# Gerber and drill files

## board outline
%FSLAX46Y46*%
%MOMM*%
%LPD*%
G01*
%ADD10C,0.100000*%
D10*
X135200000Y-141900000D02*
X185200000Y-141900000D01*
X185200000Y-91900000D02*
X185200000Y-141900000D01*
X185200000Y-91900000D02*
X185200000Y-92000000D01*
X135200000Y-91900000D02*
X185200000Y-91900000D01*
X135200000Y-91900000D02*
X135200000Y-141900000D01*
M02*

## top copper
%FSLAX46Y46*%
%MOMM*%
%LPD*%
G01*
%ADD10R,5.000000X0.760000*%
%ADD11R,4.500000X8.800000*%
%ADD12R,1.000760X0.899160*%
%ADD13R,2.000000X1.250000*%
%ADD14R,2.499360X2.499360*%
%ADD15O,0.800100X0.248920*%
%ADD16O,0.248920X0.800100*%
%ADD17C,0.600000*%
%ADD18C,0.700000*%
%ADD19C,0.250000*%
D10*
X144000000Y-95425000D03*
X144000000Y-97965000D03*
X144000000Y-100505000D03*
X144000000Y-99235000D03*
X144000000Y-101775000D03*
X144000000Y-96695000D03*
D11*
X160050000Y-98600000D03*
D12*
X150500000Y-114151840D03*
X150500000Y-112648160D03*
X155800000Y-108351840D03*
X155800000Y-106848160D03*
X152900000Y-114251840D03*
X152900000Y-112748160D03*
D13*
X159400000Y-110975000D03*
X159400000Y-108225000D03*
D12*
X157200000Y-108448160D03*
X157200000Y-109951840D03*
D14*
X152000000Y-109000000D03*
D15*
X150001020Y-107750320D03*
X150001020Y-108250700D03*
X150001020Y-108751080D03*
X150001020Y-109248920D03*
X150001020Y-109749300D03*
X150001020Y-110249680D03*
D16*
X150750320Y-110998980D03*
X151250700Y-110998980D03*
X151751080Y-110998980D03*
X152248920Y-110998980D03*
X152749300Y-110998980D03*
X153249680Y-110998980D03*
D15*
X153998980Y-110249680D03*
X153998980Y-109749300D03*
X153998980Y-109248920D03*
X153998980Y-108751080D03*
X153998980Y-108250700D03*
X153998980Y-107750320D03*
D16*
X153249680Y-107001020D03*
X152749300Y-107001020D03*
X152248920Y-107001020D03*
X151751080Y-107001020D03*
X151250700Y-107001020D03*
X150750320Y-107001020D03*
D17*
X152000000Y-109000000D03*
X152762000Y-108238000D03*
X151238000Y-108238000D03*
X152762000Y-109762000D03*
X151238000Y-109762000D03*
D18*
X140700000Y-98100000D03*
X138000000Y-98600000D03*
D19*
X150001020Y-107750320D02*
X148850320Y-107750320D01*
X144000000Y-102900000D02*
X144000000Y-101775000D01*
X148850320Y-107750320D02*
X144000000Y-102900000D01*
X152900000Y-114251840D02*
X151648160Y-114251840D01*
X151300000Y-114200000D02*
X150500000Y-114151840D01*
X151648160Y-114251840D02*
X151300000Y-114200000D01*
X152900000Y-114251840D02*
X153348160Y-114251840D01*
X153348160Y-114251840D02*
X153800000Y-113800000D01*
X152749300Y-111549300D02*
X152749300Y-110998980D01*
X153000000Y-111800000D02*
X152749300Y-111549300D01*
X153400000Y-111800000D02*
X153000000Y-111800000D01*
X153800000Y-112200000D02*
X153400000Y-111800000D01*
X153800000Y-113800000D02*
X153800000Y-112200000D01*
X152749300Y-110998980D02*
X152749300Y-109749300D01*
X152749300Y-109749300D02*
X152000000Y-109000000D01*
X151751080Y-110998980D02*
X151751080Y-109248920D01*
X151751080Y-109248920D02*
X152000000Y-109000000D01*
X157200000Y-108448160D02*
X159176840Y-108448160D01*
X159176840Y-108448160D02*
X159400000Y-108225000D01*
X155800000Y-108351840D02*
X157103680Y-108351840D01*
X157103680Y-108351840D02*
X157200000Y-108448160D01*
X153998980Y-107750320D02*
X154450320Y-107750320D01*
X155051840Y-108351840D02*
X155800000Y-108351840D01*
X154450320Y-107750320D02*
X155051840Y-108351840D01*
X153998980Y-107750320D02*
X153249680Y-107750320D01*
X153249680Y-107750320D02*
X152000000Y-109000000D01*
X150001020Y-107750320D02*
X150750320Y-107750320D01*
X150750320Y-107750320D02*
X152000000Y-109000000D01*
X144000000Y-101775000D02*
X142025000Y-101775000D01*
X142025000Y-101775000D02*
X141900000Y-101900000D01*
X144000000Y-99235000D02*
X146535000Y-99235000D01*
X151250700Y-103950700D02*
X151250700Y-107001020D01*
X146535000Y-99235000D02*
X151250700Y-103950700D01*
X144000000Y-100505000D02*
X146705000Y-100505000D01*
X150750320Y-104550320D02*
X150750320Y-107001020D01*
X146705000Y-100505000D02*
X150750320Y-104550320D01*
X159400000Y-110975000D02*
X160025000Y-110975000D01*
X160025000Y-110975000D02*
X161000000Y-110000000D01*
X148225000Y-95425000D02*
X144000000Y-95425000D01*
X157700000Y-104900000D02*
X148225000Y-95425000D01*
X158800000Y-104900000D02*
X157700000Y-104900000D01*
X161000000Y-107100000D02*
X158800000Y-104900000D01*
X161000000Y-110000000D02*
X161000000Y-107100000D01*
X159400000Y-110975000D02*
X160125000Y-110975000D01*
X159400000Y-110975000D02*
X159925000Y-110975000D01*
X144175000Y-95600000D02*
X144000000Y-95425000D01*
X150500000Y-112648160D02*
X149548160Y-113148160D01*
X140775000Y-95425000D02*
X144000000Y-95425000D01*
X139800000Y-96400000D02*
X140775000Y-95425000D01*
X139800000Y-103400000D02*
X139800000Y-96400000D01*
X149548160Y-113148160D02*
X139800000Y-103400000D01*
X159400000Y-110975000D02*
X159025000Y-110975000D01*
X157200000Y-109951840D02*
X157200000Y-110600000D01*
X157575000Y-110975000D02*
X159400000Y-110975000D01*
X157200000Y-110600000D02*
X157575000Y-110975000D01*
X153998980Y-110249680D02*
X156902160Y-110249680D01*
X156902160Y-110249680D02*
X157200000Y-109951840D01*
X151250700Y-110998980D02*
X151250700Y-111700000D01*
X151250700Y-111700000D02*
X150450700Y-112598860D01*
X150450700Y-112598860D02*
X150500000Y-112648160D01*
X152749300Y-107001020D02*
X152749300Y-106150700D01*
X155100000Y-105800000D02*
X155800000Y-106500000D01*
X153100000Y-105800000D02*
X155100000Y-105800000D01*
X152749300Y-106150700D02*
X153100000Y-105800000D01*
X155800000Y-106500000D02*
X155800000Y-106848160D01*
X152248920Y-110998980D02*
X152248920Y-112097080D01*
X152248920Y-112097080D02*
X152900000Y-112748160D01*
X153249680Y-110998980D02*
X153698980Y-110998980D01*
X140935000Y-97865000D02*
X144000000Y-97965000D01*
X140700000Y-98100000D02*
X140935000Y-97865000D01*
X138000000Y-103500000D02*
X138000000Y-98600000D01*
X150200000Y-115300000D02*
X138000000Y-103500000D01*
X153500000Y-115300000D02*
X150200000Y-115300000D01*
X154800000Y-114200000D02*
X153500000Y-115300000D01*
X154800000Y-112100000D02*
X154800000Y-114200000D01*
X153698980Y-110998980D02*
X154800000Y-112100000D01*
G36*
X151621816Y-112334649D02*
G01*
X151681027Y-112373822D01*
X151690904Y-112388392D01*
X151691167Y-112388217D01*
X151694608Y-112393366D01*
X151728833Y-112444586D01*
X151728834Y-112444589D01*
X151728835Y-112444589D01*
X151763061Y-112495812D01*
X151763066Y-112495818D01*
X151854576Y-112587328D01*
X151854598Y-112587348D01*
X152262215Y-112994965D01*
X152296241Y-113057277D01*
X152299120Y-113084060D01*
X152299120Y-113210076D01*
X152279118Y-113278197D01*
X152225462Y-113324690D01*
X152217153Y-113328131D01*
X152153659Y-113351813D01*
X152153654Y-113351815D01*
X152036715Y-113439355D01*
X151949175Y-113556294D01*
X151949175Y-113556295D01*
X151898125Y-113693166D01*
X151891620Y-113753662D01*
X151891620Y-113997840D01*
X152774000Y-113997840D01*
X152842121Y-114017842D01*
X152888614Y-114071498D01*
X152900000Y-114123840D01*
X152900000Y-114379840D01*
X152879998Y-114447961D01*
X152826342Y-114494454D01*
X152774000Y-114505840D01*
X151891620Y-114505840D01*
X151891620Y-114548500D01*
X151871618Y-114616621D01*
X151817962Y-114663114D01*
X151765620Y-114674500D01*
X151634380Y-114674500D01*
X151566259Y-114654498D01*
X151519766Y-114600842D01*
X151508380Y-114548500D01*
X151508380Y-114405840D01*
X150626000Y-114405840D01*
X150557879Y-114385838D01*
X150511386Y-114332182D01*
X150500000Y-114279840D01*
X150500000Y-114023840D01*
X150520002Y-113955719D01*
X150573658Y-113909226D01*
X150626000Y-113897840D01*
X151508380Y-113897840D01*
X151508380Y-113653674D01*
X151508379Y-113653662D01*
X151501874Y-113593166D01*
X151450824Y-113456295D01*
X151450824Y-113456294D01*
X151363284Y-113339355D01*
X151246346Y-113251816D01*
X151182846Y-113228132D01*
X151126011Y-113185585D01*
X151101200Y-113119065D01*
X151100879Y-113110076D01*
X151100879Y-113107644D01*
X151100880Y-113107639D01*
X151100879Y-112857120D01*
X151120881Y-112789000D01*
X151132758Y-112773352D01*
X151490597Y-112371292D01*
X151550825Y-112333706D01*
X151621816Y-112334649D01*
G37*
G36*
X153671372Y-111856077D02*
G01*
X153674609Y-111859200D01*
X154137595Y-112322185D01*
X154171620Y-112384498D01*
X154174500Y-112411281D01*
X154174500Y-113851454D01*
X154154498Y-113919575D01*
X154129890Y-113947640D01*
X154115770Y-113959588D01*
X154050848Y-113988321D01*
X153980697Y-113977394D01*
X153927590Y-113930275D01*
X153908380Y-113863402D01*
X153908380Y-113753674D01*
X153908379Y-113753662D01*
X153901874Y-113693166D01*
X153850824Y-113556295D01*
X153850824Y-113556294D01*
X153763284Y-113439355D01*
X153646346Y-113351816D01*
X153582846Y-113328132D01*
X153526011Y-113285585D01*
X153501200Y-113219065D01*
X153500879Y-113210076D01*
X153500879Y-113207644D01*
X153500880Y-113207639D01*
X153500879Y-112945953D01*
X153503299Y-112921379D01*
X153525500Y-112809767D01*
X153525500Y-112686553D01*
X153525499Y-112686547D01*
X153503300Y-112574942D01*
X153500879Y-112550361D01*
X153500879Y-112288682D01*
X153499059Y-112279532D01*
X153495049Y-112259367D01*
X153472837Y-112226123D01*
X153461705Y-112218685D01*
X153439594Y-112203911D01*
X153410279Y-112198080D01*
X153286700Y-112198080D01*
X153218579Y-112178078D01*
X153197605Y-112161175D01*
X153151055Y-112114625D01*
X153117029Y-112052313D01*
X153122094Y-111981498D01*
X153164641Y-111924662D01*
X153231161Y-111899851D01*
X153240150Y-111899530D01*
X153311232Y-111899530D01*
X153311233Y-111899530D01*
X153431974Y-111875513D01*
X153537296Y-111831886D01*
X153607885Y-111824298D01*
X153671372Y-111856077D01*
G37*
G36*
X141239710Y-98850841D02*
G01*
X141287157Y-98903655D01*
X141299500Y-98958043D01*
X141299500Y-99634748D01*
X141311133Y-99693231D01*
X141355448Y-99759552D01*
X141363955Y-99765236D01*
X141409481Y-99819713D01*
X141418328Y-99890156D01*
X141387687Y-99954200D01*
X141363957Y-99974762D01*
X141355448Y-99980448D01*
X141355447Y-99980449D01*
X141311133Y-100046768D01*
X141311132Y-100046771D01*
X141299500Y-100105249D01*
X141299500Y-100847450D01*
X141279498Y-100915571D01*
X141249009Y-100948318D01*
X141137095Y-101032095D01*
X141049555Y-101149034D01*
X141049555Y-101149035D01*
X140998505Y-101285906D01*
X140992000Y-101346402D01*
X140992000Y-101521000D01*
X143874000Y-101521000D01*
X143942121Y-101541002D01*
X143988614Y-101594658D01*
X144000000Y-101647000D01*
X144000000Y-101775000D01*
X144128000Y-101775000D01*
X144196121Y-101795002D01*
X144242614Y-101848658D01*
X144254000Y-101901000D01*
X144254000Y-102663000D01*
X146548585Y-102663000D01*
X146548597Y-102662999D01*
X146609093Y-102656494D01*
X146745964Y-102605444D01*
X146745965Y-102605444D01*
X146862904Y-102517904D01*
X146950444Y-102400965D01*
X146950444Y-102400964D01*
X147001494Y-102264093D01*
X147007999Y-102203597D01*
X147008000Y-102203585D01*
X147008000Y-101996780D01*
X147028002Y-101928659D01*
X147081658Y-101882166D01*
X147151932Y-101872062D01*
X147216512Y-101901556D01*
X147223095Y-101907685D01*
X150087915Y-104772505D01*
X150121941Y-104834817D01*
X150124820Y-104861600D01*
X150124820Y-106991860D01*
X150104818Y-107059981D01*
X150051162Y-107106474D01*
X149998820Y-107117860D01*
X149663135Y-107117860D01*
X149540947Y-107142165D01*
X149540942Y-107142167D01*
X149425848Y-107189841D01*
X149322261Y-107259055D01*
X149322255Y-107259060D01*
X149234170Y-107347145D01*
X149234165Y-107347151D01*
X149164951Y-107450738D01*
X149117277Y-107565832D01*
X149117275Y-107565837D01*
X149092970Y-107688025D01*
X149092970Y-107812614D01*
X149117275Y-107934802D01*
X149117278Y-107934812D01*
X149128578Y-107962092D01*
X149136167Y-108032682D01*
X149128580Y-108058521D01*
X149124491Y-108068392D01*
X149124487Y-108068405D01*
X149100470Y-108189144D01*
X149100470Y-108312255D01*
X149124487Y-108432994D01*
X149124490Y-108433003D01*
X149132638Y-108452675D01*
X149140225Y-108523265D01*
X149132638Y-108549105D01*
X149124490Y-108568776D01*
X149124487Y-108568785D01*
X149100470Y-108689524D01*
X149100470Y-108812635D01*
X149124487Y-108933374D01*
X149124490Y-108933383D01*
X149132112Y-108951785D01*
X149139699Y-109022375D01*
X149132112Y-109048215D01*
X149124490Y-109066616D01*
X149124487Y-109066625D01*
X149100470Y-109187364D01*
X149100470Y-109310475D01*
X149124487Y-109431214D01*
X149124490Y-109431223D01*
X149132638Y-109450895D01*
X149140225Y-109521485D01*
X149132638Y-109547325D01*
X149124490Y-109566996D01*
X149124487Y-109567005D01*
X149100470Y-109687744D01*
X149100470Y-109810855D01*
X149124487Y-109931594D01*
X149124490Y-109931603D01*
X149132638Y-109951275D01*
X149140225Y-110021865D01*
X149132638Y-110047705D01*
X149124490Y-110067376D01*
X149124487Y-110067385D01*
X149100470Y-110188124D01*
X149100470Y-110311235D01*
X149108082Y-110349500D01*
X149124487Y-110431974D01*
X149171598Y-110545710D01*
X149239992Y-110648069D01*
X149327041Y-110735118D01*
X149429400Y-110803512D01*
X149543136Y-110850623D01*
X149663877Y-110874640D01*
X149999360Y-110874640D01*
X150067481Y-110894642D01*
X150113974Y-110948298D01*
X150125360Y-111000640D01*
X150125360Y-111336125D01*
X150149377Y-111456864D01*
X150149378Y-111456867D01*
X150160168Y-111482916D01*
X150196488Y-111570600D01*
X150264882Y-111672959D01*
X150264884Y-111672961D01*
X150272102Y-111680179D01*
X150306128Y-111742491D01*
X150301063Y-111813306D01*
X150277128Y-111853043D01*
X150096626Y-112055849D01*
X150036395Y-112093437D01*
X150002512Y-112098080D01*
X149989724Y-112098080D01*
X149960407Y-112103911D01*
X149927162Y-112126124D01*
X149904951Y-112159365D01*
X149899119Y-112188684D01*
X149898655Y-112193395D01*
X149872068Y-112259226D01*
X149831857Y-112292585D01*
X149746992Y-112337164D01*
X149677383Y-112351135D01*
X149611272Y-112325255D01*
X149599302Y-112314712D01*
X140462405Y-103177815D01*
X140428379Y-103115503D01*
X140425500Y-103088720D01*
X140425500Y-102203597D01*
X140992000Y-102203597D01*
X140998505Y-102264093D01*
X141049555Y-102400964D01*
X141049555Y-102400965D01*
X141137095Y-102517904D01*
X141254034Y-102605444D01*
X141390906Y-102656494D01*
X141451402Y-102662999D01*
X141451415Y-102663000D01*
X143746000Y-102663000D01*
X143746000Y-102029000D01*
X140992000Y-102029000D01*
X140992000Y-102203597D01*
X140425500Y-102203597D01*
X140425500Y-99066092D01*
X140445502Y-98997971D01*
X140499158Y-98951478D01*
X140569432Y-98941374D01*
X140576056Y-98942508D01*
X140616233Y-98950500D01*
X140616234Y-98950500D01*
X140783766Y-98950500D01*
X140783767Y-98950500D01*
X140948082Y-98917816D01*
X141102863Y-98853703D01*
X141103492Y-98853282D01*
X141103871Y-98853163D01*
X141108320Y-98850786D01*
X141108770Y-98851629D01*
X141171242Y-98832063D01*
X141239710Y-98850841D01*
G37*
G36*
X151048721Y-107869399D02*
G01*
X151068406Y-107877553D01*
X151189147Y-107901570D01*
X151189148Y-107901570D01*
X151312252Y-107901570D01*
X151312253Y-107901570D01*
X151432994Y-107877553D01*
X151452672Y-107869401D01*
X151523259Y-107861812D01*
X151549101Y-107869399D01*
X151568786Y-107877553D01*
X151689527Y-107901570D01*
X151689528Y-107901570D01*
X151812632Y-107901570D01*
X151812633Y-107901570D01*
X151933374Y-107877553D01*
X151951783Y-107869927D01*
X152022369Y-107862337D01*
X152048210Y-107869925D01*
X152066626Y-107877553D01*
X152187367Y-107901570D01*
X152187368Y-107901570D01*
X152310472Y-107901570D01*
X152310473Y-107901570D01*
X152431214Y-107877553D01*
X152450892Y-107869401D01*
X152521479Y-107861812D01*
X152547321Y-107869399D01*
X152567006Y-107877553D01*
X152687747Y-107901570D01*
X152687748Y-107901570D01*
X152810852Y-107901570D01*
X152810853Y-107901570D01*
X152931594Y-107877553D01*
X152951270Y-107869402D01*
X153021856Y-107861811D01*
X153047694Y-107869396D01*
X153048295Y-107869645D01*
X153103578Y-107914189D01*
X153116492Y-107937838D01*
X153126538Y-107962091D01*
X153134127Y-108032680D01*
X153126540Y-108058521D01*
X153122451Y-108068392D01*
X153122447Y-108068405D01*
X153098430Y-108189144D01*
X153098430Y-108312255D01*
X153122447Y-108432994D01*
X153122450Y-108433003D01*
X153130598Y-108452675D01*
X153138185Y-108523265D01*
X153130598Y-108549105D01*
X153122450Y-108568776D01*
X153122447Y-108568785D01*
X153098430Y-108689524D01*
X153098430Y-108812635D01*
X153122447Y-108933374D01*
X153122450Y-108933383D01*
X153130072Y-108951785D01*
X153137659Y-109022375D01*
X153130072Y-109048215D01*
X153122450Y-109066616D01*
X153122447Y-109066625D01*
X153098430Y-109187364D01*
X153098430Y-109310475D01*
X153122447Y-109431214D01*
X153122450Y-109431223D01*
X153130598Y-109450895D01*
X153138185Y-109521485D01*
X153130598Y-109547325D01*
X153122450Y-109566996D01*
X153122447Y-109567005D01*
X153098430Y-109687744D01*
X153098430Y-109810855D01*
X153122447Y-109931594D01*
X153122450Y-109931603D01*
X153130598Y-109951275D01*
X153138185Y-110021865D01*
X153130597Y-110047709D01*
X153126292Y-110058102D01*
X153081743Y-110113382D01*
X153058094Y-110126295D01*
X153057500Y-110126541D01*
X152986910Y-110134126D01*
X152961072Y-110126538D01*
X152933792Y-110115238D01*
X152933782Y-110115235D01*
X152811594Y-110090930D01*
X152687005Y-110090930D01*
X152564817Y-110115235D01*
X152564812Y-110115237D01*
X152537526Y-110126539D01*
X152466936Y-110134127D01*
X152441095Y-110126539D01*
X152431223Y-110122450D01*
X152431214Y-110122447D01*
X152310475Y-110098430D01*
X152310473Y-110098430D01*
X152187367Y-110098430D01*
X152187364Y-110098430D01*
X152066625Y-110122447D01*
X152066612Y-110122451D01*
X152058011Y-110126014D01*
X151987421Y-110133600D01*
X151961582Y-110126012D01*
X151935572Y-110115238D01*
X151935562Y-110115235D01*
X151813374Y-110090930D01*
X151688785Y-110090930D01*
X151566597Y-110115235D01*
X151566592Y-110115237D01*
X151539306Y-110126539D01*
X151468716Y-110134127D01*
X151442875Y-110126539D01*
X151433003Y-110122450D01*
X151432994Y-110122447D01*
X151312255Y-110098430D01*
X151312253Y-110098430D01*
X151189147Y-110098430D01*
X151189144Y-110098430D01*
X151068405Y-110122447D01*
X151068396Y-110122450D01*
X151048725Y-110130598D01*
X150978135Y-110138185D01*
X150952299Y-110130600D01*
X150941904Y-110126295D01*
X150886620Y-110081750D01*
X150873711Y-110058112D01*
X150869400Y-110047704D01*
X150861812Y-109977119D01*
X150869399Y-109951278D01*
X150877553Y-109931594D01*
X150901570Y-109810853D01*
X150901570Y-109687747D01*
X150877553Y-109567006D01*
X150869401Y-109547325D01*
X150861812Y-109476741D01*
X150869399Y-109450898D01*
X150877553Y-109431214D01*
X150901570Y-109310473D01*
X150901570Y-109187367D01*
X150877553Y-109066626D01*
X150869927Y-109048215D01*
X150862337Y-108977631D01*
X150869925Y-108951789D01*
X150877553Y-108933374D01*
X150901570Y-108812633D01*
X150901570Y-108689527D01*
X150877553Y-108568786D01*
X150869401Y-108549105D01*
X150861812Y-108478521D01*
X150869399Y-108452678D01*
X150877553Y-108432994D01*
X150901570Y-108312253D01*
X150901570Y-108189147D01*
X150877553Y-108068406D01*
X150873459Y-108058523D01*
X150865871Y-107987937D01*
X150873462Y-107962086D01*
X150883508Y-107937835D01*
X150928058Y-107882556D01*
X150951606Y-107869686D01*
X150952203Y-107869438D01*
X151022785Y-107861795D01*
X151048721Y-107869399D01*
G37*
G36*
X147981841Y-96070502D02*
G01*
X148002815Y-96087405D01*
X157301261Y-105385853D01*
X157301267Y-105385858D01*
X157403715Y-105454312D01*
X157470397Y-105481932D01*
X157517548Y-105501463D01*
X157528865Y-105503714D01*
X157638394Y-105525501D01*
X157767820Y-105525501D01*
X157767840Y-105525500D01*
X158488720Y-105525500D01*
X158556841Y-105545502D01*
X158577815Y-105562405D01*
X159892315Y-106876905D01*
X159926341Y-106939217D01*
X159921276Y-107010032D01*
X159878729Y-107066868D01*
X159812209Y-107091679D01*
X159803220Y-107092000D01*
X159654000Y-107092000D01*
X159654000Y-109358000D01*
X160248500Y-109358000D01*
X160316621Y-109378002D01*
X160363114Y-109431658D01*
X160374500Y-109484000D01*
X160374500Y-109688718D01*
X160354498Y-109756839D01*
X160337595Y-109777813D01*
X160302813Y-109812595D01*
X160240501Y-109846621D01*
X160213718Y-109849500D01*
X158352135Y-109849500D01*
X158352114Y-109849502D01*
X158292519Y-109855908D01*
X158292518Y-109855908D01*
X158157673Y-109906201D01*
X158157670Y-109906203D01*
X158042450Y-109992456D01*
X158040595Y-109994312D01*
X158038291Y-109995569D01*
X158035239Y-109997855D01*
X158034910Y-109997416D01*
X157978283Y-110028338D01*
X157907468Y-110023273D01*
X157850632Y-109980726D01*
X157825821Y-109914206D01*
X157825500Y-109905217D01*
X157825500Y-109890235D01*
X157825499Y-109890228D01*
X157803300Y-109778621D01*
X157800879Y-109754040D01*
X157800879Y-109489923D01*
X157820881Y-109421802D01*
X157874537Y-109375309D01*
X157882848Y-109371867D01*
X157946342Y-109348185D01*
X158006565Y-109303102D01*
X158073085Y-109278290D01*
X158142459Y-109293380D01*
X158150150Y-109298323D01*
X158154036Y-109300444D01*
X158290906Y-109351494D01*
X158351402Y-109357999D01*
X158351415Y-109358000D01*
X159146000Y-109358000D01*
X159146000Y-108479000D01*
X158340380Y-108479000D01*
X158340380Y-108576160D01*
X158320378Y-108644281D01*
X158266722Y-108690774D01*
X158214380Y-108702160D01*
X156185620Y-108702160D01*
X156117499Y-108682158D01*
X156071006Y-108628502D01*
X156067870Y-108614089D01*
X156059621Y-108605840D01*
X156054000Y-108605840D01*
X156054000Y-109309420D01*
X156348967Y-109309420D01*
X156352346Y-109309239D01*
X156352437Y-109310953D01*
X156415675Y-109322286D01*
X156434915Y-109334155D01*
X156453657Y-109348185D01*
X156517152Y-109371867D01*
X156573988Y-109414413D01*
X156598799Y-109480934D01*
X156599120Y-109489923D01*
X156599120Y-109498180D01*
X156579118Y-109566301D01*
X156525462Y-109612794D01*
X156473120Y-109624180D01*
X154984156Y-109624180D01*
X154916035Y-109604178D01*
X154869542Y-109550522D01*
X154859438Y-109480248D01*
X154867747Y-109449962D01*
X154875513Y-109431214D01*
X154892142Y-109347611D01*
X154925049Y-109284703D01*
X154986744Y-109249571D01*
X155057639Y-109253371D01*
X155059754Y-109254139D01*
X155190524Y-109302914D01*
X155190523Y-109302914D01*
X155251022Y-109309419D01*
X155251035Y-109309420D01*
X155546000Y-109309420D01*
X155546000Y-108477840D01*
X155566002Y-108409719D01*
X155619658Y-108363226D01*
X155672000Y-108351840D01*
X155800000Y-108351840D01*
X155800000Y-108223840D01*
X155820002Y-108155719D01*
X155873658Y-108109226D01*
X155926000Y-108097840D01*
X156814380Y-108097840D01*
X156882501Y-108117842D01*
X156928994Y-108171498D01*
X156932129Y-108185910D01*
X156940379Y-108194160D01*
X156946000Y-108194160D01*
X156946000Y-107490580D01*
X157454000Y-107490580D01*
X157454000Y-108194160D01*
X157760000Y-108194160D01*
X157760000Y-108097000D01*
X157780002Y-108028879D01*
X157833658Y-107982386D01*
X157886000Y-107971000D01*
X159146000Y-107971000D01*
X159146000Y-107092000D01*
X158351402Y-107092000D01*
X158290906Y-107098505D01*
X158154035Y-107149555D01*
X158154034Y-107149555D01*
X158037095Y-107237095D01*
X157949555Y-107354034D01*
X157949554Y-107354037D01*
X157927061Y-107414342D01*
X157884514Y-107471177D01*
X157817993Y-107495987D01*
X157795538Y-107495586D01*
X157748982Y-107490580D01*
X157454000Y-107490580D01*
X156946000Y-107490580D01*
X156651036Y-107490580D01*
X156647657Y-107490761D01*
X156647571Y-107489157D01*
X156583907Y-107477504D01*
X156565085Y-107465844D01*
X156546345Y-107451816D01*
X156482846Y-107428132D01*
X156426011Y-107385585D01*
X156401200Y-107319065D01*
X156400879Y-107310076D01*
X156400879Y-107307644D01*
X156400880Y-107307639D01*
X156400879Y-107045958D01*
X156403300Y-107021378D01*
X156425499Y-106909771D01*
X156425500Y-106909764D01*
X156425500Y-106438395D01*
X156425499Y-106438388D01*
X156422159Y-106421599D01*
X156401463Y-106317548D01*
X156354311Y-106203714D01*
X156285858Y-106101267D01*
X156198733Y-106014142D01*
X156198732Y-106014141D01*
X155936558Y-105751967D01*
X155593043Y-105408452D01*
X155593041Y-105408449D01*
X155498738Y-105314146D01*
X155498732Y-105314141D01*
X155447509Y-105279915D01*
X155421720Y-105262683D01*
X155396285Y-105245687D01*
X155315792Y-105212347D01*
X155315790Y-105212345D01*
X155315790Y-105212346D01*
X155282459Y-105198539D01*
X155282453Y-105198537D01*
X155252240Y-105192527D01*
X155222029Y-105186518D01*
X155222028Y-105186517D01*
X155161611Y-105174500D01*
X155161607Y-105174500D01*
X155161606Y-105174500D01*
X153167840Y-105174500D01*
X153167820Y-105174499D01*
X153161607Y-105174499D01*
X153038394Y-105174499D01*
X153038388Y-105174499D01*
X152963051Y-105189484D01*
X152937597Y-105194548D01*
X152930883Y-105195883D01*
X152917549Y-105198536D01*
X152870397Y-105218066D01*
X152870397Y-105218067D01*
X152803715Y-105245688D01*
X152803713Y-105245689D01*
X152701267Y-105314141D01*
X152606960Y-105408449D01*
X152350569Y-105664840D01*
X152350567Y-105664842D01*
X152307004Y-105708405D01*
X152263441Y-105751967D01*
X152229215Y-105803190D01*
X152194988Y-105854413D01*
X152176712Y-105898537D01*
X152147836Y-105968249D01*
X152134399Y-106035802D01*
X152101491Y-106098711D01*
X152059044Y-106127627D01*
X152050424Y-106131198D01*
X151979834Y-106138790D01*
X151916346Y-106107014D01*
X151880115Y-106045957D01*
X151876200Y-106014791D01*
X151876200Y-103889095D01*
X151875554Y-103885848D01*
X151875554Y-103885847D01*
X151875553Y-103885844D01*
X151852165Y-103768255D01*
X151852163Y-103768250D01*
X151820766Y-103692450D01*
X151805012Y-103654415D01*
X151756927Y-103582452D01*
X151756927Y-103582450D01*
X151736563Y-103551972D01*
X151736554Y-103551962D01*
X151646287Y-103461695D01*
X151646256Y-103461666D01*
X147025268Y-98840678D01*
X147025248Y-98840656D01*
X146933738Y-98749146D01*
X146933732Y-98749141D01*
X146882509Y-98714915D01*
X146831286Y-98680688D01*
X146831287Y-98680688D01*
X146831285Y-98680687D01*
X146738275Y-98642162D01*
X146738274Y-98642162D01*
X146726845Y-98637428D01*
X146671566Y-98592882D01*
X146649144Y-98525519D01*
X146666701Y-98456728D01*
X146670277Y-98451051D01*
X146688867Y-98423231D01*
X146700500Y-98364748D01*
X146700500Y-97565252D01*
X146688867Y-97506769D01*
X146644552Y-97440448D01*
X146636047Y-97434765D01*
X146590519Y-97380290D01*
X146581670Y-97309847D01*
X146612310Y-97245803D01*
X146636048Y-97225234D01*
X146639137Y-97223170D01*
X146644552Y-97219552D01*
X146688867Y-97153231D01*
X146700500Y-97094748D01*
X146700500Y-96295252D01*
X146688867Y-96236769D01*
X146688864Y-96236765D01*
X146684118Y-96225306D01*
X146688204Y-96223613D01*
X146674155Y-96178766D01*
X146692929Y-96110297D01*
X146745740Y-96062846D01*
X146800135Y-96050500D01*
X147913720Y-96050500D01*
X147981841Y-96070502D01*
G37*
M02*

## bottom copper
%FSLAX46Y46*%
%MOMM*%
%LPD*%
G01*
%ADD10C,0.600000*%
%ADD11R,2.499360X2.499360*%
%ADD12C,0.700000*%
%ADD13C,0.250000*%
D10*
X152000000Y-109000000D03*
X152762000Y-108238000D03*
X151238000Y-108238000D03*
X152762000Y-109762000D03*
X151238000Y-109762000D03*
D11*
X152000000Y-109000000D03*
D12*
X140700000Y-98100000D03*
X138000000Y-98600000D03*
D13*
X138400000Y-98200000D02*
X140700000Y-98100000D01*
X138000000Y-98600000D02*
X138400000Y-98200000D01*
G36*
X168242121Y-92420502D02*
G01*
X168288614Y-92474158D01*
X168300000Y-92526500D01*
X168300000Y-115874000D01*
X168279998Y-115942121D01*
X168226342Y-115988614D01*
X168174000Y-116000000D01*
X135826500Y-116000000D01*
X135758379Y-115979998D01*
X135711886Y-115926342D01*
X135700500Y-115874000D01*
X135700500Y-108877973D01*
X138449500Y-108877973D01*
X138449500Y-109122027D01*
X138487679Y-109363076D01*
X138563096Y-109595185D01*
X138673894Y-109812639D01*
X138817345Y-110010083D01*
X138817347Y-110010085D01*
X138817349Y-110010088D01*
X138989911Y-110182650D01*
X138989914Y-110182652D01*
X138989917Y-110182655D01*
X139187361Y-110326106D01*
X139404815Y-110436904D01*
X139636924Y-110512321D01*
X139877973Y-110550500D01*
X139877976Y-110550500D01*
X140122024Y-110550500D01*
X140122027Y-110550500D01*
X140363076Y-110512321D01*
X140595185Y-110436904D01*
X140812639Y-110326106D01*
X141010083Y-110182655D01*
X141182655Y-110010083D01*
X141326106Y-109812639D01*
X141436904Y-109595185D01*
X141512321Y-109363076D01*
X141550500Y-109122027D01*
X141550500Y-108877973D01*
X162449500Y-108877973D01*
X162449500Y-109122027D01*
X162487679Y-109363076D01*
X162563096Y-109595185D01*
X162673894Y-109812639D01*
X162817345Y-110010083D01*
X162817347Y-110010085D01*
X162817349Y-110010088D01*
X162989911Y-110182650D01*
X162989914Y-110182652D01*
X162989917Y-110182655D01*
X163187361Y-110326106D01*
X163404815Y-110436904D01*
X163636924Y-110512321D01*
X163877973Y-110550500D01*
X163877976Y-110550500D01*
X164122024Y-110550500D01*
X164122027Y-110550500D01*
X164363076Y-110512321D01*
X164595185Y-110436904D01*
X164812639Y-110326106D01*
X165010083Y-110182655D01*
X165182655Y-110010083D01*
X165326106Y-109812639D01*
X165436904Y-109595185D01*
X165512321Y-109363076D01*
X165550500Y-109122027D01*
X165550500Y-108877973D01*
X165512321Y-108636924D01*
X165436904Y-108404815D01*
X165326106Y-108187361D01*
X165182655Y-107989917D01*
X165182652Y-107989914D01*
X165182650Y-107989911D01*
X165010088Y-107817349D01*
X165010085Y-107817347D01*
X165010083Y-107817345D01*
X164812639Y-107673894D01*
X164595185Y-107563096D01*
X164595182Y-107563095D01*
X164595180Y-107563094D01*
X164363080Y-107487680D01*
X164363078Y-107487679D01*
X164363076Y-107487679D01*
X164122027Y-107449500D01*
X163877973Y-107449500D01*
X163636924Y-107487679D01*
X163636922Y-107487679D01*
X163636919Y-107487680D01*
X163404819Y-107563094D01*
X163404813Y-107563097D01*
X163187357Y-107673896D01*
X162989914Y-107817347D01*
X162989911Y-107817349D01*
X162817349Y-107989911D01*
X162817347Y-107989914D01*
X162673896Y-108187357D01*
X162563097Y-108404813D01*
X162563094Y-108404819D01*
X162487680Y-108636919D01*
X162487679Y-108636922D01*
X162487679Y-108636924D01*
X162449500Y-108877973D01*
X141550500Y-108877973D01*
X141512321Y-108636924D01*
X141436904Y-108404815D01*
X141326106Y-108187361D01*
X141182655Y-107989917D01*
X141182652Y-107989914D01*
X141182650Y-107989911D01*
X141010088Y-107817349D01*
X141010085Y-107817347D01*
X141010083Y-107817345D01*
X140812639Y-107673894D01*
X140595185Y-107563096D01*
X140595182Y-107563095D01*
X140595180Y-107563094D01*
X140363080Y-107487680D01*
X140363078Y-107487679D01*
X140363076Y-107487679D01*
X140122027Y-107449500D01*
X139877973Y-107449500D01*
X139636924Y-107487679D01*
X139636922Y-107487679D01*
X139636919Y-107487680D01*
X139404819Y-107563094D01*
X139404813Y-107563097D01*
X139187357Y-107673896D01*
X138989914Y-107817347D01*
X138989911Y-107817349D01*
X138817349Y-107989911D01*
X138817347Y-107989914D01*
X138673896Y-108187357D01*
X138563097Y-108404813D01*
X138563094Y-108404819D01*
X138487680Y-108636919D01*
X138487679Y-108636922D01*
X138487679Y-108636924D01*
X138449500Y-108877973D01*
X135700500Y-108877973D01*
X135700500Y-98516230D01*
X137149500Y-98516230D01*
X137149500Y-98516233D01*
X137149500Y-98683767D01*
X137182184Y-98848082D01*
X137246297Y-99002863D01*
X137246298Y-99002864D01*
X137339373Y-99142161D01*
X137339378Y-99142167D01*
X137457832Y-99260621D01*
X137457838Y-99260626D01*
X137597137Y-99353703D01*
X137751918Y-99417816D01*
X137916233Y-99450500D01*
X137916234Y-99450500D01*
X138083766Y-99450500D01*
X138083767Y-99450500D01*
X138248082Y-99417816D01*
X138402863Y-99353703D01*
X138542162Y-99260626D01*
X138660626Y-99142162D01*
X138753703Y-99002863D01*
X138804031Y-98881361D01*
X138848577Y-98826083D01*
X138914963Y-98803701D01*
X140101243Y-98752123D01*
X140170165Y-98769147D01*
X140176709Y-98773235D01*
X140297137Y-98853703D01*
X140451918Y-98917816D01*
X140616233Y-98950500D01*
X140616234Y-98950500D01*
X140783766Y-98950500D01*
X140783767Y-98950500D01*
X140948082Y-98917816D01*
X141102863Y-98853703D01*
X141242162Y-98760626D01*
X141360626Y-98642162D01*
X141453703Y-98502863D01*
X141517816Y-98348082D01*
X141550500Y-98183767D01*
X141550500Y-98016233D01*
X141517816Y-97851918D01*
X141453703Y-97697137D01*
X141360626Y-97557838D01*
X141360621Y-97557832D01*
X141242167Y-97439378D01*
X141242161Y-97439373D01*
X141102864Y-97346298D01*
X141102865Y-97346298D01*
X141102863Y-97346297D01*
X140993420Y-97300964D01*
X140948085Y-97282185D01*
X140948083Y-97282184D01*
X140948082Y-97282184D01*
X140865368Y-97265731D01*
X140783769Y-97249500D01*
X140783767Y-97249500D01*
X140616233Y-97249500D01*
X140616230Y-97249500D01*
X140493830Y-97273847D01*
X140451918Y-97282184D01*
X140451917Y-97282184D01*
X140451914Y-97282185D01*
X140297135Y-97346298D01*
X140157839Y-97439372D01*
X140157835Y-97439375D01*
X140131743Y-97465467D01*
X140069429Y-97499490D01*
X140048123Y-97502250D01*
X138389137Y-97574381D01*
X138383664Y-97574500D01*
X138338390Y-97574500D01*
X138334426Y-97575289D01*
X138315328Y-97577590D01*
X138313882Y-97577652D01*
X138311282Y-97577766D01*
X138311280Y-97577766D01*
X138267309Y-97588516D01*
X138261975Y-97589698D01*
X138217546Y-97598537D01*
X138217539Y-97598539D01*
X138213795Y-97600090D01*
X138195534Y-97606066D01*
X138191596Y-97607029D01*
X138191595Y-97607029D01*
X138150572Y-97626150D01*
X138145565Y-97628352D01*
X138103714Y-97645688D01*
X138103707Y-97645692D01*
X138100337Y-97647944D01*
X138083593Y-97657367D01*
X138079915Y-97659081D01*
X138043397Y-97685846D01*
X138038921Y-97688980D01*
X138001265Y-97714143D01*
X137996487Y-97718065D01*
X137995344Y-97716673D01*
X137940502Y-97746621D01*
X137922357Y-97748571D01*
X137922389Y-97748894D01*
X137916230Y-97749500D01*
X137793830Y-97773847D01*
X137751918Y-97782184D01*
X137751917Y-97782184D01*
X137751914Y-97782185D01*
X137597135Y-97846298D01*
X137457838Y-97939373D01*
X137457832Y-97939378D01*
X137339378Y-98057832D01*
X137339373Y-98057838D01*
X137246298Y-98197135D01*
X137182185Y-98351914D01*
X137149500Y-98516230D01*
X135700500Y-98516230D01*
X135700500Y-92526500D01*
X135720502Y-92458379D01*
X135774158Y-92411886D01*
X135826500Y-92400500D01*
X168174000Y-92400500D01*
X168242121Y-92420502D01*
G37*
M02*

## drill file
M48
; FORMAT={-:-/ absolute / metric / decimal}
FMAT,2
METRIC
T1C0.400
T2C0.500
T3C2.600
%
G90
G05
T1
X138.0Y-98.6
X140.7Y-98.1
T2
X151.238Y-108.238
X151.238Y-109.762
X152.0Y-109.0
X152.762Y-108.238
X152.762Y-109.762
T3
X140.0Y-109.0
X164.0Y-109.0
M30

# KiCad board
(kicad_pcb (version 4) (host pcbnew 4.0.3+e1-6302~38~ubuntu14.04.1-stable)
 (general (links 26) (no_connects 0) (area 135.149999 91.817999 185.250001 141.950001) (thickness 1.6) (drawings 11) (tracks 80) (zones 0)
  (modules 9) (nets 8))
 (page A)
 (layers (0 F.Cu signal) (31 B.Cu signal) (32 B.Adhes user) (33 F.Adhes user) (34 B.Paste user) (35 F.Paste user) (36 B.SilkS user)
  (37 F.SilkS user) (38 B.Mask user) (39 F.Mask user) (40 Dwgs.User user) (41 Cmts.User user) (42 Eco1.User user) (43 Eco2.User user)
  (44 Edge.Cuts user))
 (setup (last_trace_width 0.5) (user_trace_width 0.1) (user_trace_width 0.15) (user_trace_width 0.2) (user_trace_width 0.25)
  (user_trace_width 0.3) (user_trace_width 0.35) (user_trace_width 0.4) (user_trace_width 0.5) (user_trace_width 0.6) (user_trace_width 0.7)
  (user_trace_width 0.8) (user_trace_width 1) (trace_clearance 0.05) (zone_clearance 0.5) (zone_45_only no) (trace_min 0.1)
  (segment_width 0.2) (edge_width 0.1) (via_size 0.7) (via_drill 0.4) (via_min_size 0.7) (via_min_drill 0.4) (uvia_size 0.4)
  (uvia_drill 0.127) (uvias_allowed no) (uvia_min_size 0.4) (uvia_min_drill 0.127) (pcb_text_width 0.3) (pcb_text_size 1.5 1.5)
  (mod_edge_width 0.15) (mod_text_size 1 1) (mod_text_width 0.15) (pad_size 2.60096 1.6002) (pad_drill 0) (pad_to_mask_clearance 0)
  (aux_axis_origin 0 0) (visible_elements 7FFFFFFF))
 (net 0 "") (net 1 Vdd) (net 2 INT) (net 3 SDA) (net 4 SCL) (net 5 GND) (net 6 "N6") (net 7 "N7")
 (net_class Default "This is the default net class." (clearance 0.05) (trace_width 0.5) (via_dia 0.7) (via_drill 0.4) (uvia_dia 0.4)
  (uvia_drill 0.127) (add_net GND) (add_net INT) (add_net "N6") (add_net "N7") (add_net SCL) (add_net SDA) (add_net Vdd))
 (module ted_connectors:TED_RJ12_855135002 (layer F.Cu) (at 151.9 98.6 270)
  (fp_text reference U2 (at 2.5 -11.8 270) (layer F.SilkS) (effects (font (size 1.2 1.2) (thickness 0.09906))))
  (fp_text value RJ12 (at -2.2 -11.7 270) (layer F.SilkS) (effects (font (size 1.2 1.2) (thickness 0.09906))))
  (pad 6 smd rect (at -3.175 7.9 270) (size 0.76 5) (layers F.Cu F.Paste F.Mask) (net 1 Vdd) (clearance 0.2))
  (pad 4 smd rect (at -0.635 7.9 270) (size 0.76 5) (layers F.Cu F.Paste F.Mask) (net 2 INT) (clearance 0.2))
  (pad 2 smd rect (at 1.905 7.9 270) (size 0.76 5) (layers F.Cu F.Paste F.Mask) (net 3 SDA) (clearance 0.2))
  (pad 3 smd rect (at 0.635 7.9 270) (size 0.76 5) (layers F.Cu F.Paste F.Mask) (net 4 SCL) (clearance 0.2))
  (pad 1 smd rect (at 3.175 7.9 270) (size 0.76 5) (layers F.Cu F.Paste F.Mask) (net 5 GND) (clearance 0.2))
  (pad 5 smd rect (at -1.905 7.9 270) (size 0.76 5) (layers F.Cu F.Paste F.Mask) (clearance 0.2))
  (pad PAD smd rect (at 0 -8.15 270) (size 8.8 4.5) (layers F.Cu F.Paste F.Mask)))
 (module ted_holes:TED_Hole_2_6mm (layer F.Cu) (at 140 109)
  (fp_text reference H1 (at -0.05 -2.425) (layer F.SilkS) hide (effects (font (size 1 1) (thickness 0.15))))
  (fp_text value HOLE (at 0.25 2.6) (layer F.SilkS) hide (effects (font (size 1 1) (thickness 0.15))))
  (pad "" np_thru_hole circle (at 0 0) (size 2.6 2.6) (drill 2.6) (layers *.Cu *.Mask F.SilkS)))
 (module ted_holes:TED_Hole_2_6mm (layer F.Cu) (at 164 109)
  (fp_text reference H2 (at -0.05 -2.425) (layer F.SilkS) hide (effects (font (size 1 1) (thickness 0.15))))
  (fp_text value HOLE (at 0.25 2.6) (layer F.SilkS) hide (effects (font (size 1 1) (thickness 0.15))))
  (pad "" np_thru_hole circle (at 0 0) (size 2.6 2.6) (drill 2.6) (layers *.Cu *.Mask F.SilkS)))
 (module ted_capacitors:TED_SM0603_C (layer F.Cu) (at 150.5 113.4 270)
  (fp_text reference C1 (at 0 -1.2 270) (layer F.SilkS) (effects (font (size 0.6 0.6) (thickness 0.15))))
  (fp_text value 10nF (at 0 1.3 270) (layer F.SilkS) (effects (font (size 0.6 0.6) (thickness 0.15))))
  (pad 2 smd rect (at 0.75184 0 270) (size 0.89916 1.00076) (layers F.Cu F.Paste F.Mask) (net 5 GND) (clearance 0.1))
  (pad 1 smd rect (at -0.75184 0 270) (size 0.89916 1.00076) (layers F.Cu F.Paste F.Mask) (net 1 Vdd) (clearance 0.1)))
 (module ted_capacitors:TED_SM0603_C (layer F.Cu) (at 155.8 107.6 270)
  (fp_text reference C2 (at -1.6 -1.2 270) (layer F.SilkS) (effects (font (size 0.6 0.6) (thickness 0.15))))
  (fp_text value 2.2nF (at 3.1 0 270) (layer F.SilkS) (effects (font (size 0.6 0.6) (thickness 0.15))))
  (pad 2 smd rect (at 0.75184 0 270) (size 0.89916 1.00076) (layers F.Cu F.Paste F.Mask) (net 5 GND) (clearance 0.1))
  (pad 1 smd rect (at -0.75184 0 270) (size 0.89916 1.00076) (layers F.Cu F.Paste F.Mask) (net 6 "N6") (clearance 0.1)))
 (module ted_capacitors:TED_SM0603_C (layer F.Cu) (at 152.9 113.5 270)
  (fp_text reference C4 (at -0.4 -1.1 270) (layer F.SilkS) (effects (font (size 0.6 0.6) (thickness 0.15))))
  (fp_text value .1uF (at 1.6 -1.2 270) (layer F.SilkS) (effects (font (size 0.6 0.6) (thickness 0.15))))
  (pad 2 smd rect (at 0.75184 0 270) (size 0.89916 1.00076) (layers F.Cu F.Paste F.Mask) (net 5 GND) (clearance 0.1))
  (pad 1 smd rect (at -0.75184 0 270) (size 0.89916 1.00076) (layers F.Cu F.Paste F.Mask) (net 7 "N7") (clearance 0.1)))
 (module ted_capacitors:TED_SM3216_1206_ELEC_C (layer F.Cu) (at 159.4 109.6 90)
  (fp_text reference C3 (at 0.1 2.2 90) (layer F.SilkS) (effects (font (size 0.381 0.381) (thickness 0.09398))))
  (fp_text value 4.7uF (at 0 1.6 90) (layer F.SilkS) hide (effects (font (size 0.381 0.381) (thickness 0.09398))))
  (pad 1 smd rect (at -1.375 0 90) (size 1.25 2) (layers F.Cu F.Paste F.Mask) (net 1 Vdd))
  (pad 2 smd rect (at 1.375 0 90) (size 1.25 2) (layers F.Cu F.Paste F.Mask) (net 5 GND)))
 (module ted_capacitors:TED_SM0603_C (layer F.Cu) (at 157.2 109.2 90)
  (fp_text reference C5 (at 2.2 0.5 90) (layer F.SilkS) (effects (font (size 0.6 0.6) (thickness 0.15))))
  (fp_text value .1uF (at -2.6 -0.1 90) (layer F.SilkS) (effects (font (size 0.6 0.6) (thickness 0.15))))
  (pad 2 smd rect (at 0.75184 0 90) (size 0.89916 1.00076) (layers F.Cu F.Paste F.Mask) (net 5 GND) (clearance 0.1))
  (pad 1 smd rect (at -0.75184 0 90) (size 0.89916 1.00076) (layers F.Cu F.Paste F.Mask) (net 1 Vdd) (clearance 0.1)))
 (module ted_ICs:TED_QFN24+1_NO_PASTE (layer F.Cu) (at 152 109)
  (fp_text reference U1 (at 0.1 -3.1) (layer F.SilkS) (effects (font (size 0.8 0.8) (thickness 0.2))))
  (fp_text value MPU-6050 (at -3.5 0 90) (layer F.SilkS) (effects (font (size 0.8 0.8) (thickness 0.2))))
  (pad 25 smd rect (at 0 0 270) (size 2.49936 2.49936) (layers F.Cu F.Mask) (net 5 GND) (zone_connect 2))
  (pad 1 smd oval (at -1.99898 -1.24968) (size 0.8001 0.24892) (layers F.Cu F.Paste F.Mask) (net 5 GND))
  (pad 2 smd oval (at -1.99898 -0.7493) (size 0.8001 0.24892) (layers F.Cu F.Paste F.Mask))
  (pad 3 smd oval (at -1.99898 -0.24892) (size 0.8001 0.24892) (layers F.Cu F.Paste F.Mask))
  (pad 4 smd oval (at -1.99898 0.24892) (size 0.8001 0.24892) (layers F.Cu F.Paste F.Mask))
  (pad 5 smd oval (at -1.99898 0.7493) (size 0.8001 0.24892) (layers F.Cu F.Paste F.Mask))
  (pad 6 smd oval (at -1.99898 1.24968) (size 0.8001 0.24892) (layers F.Cu F.Paste F.Mask))
  (pad 7 smd oval (at -1.24968 1.99898 90) (size 0.8001 0.24892) (layers F.Cu F.Paste F.Mask))
  (pad 8 smd oval (at -0.7493 1.99898 90) (size 0.8001 0.24892) (layers F.Cu F.Paste F.Mask) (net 1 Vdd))
  (pad 9 smd oval (at -0.24892 1.99898 90) (size 0.8001 0.24892) (layers F.Cu F.Paste F.Mask) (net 5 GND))
  (pad 10 smd oval (at 0.24892 1.99898 90) (size 0.8001 0.24892) (layers F.Cu F.Paste F.Mask) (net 7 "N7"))
  (pad 11 smd oval (at 0.7493 1.99898 90) (size 0.8001 0.24892) (layers F.Cu F.Paste F.Mask) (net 5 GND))
  (pad 12 smd oval (at 1.24968 1.99898 90) (size 0.8001 0.24892) (layers F.Cu F.Paste F.Mask) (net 2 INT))
  (pad 13 smd oval (at 1.99898 1.24968 180) (size 0.8001 0.24892) (layers F.Cu F.Paste F.Mask) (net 1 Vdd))
  (pad 14 smd oval (at 1.99898 0.7493 180) (size 0.8001 0.24892) (layers F.Cu F.Paste F.Mask))
  (pad 15 smd oval (at 1.99898 0.24892 180) (size 0.8001 0.24892) (layers F.Cu F.Paste F.Mask))
  (pad 16 smd oval (at 1.99898 -0.24892 180) (size 0.8001 0.24892) (layers F.Cu F.Paste F.Mask))
  (pad 17 smd oval (at 1.99898 -0.7493 180) (size 0.8001 0.24892) (layers F.Cu F.Paste F.Mask))
  (pad 18 smd oval (at 1.99898 -1.24968 180) (size 0.8001 0.24892) (layers F.Cu F.Paste F.Mask) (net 5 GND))
  (pad 19 smd oval (at 1.24968 -1.99898 270) (size 0.8001 0.24892) (layers F.Cu F.Paste F.Mask))
  (pad 20 smd oval (at 0.7493 -1.99898 270) (size 0.8001 0.24892) (layers F.Cu F.Paste F.Mask) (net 6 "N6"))
  (pad 21 smd oval (at 0.24892 -1.99898 270) (size 0.8001 0.24892) (layers F.Cu F.Paste F.Mask))
  (pad 22 smd oval (at -0.24892 -1.99898 270) (size 0.8001 0.24892) (layers F.Cu F.Paste F.Mask))
  (pad 23 smd oval (at -0.7493 -1.99898 270) (size 0.8001 0.24892) (layers F.Cu F.Paste F.Mask) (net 4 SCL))
  (pad 24 smd oval (at -1.24968 -1.99898 270) (size 0.8001 0.24892) (layers F.Cu F.Paste F.Mask) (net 3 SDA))
  (pad 25 thru_hole circle (at 0 0 270) (size 0.6 0.6) (drill 0.5) (layers *.Cu) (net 5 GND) (zone_connect 2))
  (pad 25 thru_hole circle (at 0.762 -0.762 270) (size 0.6 0.6) (drill 0.5) (layers *.Cu) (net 5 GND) (zone_connect 2))
  (pad 25 thru_hole circle (at -0.762 -0.762 270) (size 0.6 0.6) (drill 0.5) (layers *.Cu) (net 5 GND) (zone_connect 2))
  (pad 25 thru_hole circle (at 0.762 0.762 270) (size 0.6 0.6) (drill 0.5) (layers *.Cu) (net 5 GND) (zone_connect 2))
  (pad 25 thru_hole circle (at -0.762 0.762 270) (size 0.6 0.6) (drill 0.5) (layers *.Cu) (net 5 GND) (zone_connect 2))
  (pad 25 smd rect (at 0 0 270) (size 2.49936 2.49936) (layers B.Cu B.Mask) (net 5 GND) (zone_connect 2)))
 (gr_line (start 135.2 141.9) (end 185.2 141.9) (angle 90) (layer Edge.Cuts) (width 0.1))
 (gr_line (start 185.2 91.9) (end 185.2 141.9) (angle 90) (layer Edge.Cuts) (width 0.1))
 (gr_line (start 185.2 91.9) (end 185.2 92) (angle 90) (layer Edge.Cuts) (width 0.1))
 (gr_line (start 135.2 91.9) (end 185.2 91.9) (angle 90) (layer Edge.Cuts) (width 0.1))
 (gr_line (start 135.2 91.9) (end 135.2 141.9) (angle 90) (layer Edge.Cuts) (width 0.1))
 (segment (start 150.00102 107.75032) (end 148.85032 107.75032) (width 0.25) (layer F.Cu) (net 5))
 (segment (start 144 102.9) (end 144 101.775) (width 0.25) (layer F.Cu) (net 5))
 (segment (start 148.85032 107.75032) (end 144 102.9) (width 0.25) (layer F.Cu) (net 5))
 (segment (start 152.9 114.25184) (end 151.64816 114.25184) (width 0.25) (layer F.Cu) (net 5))
 (segment (start 151.3 114.2) (end 150.5 114.15184) (width 0.25) (layer F.Cu) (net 5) (status 20))
 (segment (start 151.64816 114.25184) (end 151.3 114.2) (width 0.25) (layer F.Cu) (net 5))
 (segment (start 152.9 114.25184) (end 153.34816 114.25184) (width 0.25) (layer F.Cu) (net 5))
 (segment (start 153.34816 114.25184) (end 153.8 113.8) (width 0.25) (layer F.Cu) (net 5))
 (segment (start 152.7493 111.5493) (end 152.7493 110.99898) (width 0.25) (layer F.Cu) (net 5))
 (segment (start 153 111.8) (end 152.7493 111.5493) (width 0.25) (layer F.Cu) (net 5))
 (segment (start 153.4 111.8) (end 153 111.8) (width 0.25) (layer F.Cu) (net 5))
 (segment (start 153.8 112.2) (end 153.4 111.8) (width 0.25) (layer F.Cu) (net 5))
 (segment (start 153.8 113.8) (end 153.8 112.2) (width 0.25) (layer F.Cu) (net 5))
 (segment (start 152.7493 110.99898) (end 152.7493 109.7493) (width 0.25) (layer F.Cu) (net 5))
 (segment (start 152.7493 109.7493) (end 152 109) (width 0.25) (layer F.Cu) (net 5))
 (segment (start 151.75108 110.99898) (end 151.75108 109.24892) (width 0.25) (layer F.Cu) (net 5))
 (segment (start 151.75108 109.24892) (end 152 109) (width 0.25) (layer F.Cu) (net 5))
 (segment (start 157.2 108.44816) (end 159.17684 108.44816) (width 0.25) (layer F.Cu) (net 5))
 (segment (start 159.17684 108.44816) (end 159.4 108.225) (width 0.25) (layer F.Cu) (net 5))
 (segment (start 155.8 108.35184) (end 157.10368 108.35184) (width 0.25) (layer F.Cu) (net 5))
 (segment (start 157.10368 108.35184) (end 157.2 108.44816) (width 0.25) (layer F.Cu) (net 5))
 (segment (start 153.99898 107.75032) (end 154.45032 107.75032) (width 0.25) (layer F.Cu) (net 5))
 (segment (start 155.05184 108.35184) (end 155.8 108.35184) (width 0.25) (layer F.Cu) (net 5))
 (segment (start 154.45032 107.75032) (end 155.05184 108.35184) (width 0.25) (layer F.Cu) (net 5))
 (segment (start 153.99898 107.75032) (end 153.24968 107.75032) (width 0.25) (layer F.Cu) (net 5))
 (segment (start 153.24968 107.75032) (end 152 109) (width 0.25) (layer F.Cu) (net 5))
 (segment (start 150.00102 107.75032) (end 150.75032 107.75032) (width 0.25) (layer F.Cu) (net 5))
 (segment (start 150.75032 107.75032) (end 152 109) (width 0.25) (layer F.Cu) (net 5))
 (segment (start 144 101.775) (end 142.025 101.775) (width 0.25) (layer F.Cu) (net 5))
 (segment (start 142.025 101.775) (end 141.9 101.9) (width 0.25) (layer F.Cu) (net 5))
 (segment (start 144 99.235) (end 146.535 99.235) (width 0.25) (layer F.Cu) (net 4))
 (segment (start 151.2507 103.9507) (end 151.2507 107.00102) (width 0.25) (layer F.Cu) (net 4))
 (segment (start 146.535 99.235) (end 151.2507 103.9507) (width 0.25) (layer F.Cu) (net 4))
 (segment (start 144 100.505) (end 146.705 100.505) (width 0.25) (layer F.Cu) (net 3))
 (segment (start 150.75032 104.55032) (end 150.75032 107.00102) (width 0.25) (layer F.Cu) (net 3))
 (segment (start 146.705 100.505) (end 150.75032 104.55032) (width 0.25) (layer F.Cu) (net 3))
 (segment (start 159.4 110.975) (end 160.025 110.975) (width 0.25) (layer F.Cu) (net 1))
 (segment (start 160.025 110.975) (end 161 110) (width 0.25) (layer F.Cu) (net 1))
 (segment (start 148.225 95.425) (end 144 95.425) (width 0.25) (layer F.Cu) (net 1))
 (segment (start 157.7 104.9) (end 148.225 95.425) (width 0.25) (layer F.Cu) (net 1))
 (segment (start 158.8 104.9) (end 157.7 104.9) (width 0.25) (layer F.Cu) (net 1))
 (segment (start 161 107.1) (end 158.8 104.9) (width 0.25) (layer F.Cu) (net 1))
 (segment (start 161 110) (end 161 107.1) (width 0.25) (layer F.Cu) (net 1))
 (segment (start 159.4 110.975) (end 160.125 110.975) (width 0.25) (layer F.Cu) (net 1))
 (segment (start 159.4 110.975) (end 159.925 110.975) (width 0.25) (layer F.Cu) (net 1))
 (segment (start 144.175 95.6) (end 144 95.425) (width 0.25) (layer F.Cu) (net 1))
 (segment (start 150.5 112.64816) (end 149.54816 113.14816) (width 0.25) (layer F.Cu) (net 1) (status 10))
 (segment (start 140.775 95.425) (end 144 95.425) (width 0.25) (layer F.Cu) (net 1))
 (segment (start 139.8 96.4) (end 140.775 95.425) (width 0.25) (layer F.Cu) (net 1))
 (segment (start 139.8 103.4) (end 139.8 96.4) (width 0.25) (layer F.Cu) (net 1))
 (segment (start 149.54816 113.14816) (end 139.8 103.4) (width 0.25) (layer F.Cu) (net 1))
 (segment (start 159.4 110.975) (end 159.025 110.975) (width 0.25) (layer F.Cu) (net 1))
 (segment (start 157.2 109.95184) (end 157.2 110.6) (width 0.25) (layer F.Cu) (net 1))
 (segment (start 157.575 110.975) (end 159.4 110.975) (width 0.25) (layer F.Cu) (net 1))
 (segment (start 157.2 110.6) (end 157.575 110.975) (width 0.25) (layer F.Cu) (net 1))
 (segment (start 153.99898 110.24968) (end 156.90216 110.24968) (width 0.25) (layer F.Cu) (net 1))
 (segment (start 156.90216 110.24968) (end 157.2 109.95184) (width 0.25) (layer F.Cu) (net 1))
 (segment (start 151.2507 110.99898) (end 151.2507 111.7) (width 0.25) (layer F.Cu) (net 1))
 (segment (start 151.2507 111.7) (end 150.4507 112.59886) (width 0.25) (layer F.Cu) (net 1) (status 20))
 (segment (start 150.4507 112.59886) (end 150.5 112.64816) (width 0.25) (layer F.Cu) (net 1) (status 30))
 (segment (start 152.7493 107.00102) (end 152.7493 106.1507) (width 0.25) (layer F.Cu) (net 6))
 (segment (start 155.1 105.8) (end 155.8 106.5) (width 0.25) (layer F.Cu) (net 6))
 (segment (start 153.1 105.8) (end 155.1 105.8) (width 0.25) (layer F.Cu) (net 6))
 (segment (start 152.7493 106.1507) (end 153.1 105.8) (width 0.25) (layer F.Cu) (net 6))
 (segment (start 155.8 106.5) (end 155.8 106.84816) (width 0.25) (layer F.Cu) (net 6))
 (segment (start 152.24892 110.99898) (end 152.24892 112.09708) (width 0.25) (layer F.Cu) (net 7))
 (segment (start 152.24892 112.09708) (end 152.9 112.74816) (width 0.25) (layer F.Cu) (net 7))
 (segment (start 153.24968 110.99898) (end 153.69898 110.99898) (width 0.25) (layer F.Cu) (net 2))
 (segment (start 140.935 97.865) (end 144 97.965) (width 0.25) (layer F.Cu) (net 2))
 (segment (start 140.7 98.1) (end 140.935 97.865) (width 0.25) (layer F.Cu) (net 2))
 (via (at 140.7 98.1) (size 0.7) (drill 0.4) (layers F.Cu B.Cu) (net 2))
 (segment (start 138.4 98.2) (end 140.7 98.1) (width 0.25) (layer B.Cu) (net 2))
 (segment (start 138 98.6) (end 138.4 98.2) (width 0.25) (layer B.Cu) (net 2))
 (via (at 138 98.6) (size 0.7) (drill 0.4) (layers F.Cu B.Cu) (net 2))
 (segment (start 138 103.5) (end 138 98.6) (width 0.25) (layer F.Cu) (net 2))
 (segment (start 150.2 115.3) (end 138 103.5) (width 0.25) (layer F.Cu) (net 2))
 (segment (start 153.5 115.3) (end 150.2 115.3) (width 0.25) (layer F.Cu) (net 2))
 (segment (start 154.8 114.2) (end 153.5 115.3) (width 0.25) (layer F.Cu) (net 2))
 (segment (start 154.8 112.1) (end 154.8 114.2) (width 0.25) (layer F.Cu) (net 2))
 (segment (start 153.69898 110.99898) (end 154.8 112.1) (width 0.25) (layer F.Cu) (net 2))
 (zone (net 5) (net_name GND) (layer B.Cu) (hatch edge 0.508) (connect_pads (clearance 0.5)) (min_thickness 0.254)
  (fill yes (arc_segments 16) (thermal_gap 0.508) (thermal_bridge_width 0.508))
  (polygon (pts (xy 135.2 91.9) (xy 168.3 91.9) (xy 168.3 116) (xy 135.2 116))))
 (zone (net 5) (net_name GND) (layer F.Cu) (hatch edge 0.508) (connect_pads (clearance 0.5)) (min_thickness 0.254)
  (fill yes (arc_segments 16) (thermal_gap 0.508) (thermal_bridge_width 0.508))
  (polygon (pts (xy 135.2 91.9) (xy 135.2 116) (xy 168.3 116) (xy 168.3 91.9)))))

